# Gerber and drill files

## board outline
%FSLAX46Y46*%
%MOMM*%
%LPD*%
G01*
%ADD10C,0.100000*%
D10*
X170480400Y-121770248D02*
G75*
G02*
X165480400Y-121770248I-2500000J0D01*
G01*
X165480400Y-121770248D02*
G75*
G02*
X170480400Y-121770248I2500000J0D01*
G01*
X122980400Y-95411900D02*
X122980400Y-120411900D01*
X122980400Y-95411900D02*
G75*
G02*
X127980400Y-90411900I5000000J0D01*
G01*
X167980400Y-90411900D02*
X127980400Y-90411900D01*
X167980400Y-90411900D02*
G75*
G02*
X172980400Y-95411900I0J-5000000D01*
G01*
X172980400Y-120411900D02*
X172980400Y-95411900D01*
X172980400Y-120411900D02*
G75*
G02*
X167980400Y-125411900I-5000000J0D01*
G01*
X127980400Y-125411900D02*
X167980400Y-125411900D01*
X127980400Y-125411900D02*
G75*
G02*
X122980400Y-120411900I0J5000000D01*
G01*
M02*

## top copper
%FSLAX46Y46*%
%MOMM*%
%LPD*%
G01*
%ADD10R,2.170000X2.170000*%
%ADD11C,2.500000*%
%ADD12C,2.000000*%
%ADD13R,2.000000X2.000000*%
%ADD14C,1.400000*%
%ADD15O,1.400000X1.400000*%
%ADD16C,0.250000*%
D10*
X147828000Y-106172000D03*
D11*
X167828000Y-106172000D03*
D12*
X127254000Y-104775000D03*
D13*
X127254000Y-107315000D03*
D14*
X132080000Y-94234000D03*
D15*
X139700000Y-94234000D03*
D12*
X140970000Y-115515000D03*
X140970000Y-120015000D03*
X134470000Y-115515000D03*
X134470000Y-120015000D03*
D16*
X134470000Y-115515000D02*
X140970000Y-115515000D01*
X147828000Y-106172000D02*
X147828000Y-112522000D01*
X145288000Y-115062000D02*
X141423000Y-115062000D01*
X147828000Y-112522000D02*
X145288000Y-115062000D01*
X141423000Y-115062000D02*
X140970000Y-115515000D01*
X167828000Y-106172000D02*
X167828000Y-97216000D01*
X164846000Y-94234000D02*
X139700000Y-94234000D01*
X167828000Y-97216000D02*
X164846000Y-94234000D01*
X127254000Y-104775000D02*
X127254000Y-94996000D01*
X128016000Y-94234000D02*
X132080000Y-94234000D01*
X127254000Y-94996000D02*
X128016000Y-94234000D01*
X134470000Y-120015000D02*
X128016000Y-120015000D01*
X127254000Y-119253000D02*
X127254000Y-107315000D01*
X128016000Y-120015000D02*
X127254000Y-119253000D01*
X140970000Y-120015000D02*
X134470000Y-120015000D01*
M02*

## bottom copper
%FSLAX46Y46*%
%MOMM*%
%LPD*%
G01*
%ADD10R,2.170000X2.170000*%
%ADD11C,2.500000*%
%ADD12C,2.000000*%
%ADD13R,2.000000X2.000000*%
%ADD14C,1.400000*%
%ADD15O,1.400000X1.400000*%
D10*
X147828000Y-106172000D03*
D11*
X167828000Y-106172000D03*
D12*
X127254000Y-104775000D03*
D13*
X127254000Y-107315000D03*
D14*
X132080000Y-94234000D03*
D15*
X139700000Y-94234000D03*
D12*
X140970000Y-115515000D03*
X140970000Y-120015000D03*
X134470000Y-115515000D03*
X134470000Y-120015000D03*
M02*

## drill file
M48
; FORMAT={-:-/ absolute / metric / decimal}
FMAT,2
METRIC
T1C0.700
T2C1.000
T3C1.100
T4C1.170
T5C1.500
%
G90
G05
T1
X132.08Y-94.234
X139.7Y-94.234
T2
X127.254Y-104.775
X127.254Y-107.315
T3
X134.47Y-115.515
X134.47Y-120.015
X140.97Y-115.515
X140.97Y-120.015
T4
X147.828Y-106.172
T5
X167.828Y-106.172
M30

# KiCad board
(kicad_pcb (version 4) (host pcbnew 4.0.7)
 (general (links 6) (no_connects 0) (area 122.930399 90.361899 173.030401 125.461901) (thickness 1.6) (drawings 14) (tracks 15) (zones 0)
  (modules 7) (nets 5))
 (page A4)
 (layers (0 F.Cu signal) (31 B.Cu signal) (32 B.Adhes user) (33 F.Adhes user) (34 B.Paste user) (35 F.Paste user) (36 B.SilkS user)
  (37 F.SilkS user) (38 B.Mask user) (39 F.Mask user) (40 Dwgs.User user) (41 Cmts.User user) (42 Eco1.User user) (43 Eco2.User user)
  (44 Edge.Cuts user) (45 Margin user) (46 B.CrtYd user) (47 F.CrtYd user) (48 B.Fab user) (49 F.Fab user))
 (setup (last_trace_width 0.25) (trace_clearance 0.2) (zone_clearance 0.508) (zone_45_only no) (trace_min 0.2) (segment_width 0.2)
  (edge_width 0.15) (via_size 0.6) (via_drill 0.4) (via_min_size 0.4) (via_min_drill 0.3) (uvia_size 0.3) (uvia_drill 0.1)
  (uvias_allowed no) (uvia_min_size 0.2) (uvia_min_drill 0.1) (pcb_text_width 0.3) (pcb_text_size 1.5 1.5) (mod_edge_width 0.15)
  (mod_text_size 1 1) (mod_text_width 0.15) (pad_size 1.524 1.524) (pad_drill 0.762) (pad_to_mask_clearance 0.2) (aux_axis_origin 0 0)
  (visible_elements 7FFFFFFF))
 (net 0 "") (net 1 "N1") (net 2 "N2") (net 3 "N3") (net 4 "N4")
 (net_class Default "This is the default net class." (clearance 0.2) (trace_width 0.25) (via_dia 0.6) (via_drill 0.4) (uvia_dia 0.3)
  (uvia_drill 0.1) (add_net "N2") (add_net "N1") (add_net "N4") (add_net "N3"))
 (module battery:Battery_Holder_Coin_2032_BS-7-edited (layer F.Cu) (at 147.828 106.172)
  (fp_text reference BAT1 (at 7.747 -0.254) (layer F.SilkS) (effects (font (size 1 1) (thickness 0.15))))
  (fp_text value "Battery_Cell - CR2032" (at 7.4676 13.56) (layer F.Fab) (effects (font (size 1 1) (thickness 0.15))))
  (pad 2 thru_hole rect (at 0 0) (size 2.17 2.17) (drill 1.17) (layers *.Cu *.Mask) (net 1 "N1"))
  (pad 1 thru_hole circle (at 20 0) (size 2.5 2.5) (drill 1.5) (layers *.Cu *.Mask) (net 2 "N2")))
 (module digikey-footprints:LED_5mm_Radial (layer F.Cu) (at 127.254 104.775 90)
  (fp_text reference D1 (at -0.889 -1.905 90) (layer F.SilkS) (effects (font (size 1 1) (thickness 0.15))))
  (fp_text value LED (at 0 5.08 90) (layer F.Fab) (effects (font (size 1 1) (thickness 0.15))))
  (pad 2 thru_hole circle (at 0 0 90) (size 2 2) (drill 1) (layers *.Cu *.Mask) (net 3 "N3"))
  (pad 1 thru_hole rect (at -2.54 0 90) (size 2 2) (drill 1) (layers *.Cu *.Mask) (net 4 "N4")))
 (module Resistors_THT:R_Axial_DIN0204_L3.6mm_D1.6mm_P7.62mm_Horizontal (layer F.Cu) (at 132.08 94.234)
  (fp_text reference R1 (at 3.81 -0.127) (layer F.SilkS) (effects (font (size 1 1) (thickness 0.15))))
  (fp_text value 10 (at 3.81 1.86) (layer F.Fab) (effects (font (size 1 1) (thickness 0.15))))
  (pad 1 thru_hole circle (at 0 0) (size 1.4 1.4) (drill 0.7) (layers *.Cu *.Mask) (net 3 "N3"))
  (pad 2 thru_hole oval (at 7.62 0) (size 1.4 1.4) (drill 0.7) (layers *.Cu *.Mask) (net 2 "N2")))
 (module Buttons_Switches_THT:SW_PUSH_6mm (layer F.Cu) (at 140.97 120.015 180)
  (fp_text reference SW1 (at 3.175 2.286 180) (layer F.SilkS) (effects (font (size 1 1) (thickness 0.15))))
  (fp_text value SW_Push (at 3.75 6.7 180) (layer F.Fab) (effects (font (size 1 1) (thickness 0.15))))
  (pad 2 thru_hole circle (at 0 4.5 270) (size 2 2) (drill 1.1) (layers *.Cu *.Mask) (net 1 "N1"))
  (pad 1 thru_hole circle (at 0 0 270) (size 2 2) (drill 1.1) (layers *.Cu *.Mask) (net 4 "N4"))
  (pad 2 thru_hole circle (at 6.5 4.5 270) (size 2 2) (drill 1.1) (layers *.Cu *.Mask) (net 1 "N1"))
  (pad 1 thru_hole circle (at 6.5 0 270) (size 2 2) (drill 1.1) (layers *.Cu *.Mask) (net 4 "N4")))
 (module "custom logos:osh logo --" (layer F.Cu) (at 131.064 99.568)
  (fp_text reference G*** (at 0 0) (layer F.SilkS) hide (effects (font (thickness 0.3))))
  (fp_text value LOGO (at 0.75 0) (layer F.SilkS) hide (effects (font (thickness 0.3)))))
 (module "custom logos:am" (layer F.Cu) (at 129.667 114.935)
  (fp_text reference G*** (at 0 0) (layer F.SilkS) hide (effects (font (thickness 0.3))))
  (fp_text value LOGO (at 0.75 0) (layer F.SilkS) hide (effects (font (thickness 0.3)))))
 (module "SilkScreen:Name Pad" (layer F.Cu) (at 139.827 104.394 90)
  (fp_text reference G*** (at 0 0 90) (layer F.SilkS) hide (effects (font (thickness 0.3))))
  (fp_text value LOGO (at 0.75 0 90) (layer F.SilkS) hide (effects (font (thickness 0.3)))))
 (gr_circle (center 167.9804 121.770248) (end 167.9804 119.270248) (layer Edge.Cuts) (width 0.1))
 (gr_line (start 122.9804 95.4119) (end 122.9804 120.4119) (layer Edge.Cuts) (width 0.1))
 (gr_arc (start 127.9804 95.4119) (end 122.9804 95.4119) (angle 90) (layer Edge.Cuts) (width 0.1))
 (gr_line (start 167.9804 90.4119) (end 127.9804 90.4119) (layer Edge.Cuts) (width 0.1))
 (gr_arc (start 167.9804 95.4119) (end 167.9804 90.4119) (angle 90) (layer Edge.Cuts) (width 0.1))
 (gr_line (start 172.9804 120.4119) (end 172.9804 95.4119) (layer Edge.Cuts) (width 0.1))
 (gr_arc (start 167.9804 120.4119) (end 172.9804 120.4119) (angle 90) (layer Edge.Cuts) (width 0.1))
 (gr_line (start 127.9804 125.4119) (end 167.9804 125.4119) (layer Edge.Cuts) (width 0.1))
 (gr_arc (start 127.9804 120.4119) (end 127.9804 125.4119) (angle 90) (layer Edge.Cuts) (width 0.1))
 (segment (start 134.47 115.515) (end 140.97 115.515) (width 0.25) (layer F.Cu) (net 1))
 (segment (start 147.828 106.172) (end 147.828 112.522) (width 0.25) (layer F.Cu) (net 1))
 (segment (start 145.288 115.062) (end 141.423 115.062) (width 0.25) (layer F.Cu) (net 1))
 (segment (start 147.828 112.522) (end 145.288 115.062) (width 0.25) (layer F.Cu) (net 1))
 (segment (start 141.423 115.062) (end 140.97 115.515) (width 0.25) (layer F.Cu) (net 1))
 (segment (start 167.828 106.172) (end 167.828 97.216) (width 0.25) (layer F.Cu) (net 2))
 (segment (start 164.846 94.234) (end 139.7 94.234) (width 0.25) (layer F.Cu) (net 2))
 (segment (start 167.828 97.216) (end 164.846 94.234) (width 0.25) (layer F.Cu) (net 2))
 (segment (start 127.254 104.775) (end 127.254 94.996) (width 0.25) (layer F.Cu) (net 3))
 (segment (start 128.016 94.234) (end 132.08 94.234) (width 0.25) (layer F.Cu) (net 3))
 (segment (start 127.254 94.996) (end 128.016 94.234) (width 0.25) (layer F.Cu) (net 3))
 (segment (start 134.47 120.015) (end 128.016 120.015) (width 0.25) (layer F.Cu) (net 4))
 (segment (start 127.254 119.253) (end 127.254 107.315) (width 0.25) (layer F.Cu) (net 4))
 (segment (start 128.016 120.015) (end 127.254 119.253) (width 0.25) (layer F.Cu) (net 4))
 (segment (start 140.97 120.015) (end 134.47 120.015) (width 0.25) (layer F.Cu) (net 4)))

